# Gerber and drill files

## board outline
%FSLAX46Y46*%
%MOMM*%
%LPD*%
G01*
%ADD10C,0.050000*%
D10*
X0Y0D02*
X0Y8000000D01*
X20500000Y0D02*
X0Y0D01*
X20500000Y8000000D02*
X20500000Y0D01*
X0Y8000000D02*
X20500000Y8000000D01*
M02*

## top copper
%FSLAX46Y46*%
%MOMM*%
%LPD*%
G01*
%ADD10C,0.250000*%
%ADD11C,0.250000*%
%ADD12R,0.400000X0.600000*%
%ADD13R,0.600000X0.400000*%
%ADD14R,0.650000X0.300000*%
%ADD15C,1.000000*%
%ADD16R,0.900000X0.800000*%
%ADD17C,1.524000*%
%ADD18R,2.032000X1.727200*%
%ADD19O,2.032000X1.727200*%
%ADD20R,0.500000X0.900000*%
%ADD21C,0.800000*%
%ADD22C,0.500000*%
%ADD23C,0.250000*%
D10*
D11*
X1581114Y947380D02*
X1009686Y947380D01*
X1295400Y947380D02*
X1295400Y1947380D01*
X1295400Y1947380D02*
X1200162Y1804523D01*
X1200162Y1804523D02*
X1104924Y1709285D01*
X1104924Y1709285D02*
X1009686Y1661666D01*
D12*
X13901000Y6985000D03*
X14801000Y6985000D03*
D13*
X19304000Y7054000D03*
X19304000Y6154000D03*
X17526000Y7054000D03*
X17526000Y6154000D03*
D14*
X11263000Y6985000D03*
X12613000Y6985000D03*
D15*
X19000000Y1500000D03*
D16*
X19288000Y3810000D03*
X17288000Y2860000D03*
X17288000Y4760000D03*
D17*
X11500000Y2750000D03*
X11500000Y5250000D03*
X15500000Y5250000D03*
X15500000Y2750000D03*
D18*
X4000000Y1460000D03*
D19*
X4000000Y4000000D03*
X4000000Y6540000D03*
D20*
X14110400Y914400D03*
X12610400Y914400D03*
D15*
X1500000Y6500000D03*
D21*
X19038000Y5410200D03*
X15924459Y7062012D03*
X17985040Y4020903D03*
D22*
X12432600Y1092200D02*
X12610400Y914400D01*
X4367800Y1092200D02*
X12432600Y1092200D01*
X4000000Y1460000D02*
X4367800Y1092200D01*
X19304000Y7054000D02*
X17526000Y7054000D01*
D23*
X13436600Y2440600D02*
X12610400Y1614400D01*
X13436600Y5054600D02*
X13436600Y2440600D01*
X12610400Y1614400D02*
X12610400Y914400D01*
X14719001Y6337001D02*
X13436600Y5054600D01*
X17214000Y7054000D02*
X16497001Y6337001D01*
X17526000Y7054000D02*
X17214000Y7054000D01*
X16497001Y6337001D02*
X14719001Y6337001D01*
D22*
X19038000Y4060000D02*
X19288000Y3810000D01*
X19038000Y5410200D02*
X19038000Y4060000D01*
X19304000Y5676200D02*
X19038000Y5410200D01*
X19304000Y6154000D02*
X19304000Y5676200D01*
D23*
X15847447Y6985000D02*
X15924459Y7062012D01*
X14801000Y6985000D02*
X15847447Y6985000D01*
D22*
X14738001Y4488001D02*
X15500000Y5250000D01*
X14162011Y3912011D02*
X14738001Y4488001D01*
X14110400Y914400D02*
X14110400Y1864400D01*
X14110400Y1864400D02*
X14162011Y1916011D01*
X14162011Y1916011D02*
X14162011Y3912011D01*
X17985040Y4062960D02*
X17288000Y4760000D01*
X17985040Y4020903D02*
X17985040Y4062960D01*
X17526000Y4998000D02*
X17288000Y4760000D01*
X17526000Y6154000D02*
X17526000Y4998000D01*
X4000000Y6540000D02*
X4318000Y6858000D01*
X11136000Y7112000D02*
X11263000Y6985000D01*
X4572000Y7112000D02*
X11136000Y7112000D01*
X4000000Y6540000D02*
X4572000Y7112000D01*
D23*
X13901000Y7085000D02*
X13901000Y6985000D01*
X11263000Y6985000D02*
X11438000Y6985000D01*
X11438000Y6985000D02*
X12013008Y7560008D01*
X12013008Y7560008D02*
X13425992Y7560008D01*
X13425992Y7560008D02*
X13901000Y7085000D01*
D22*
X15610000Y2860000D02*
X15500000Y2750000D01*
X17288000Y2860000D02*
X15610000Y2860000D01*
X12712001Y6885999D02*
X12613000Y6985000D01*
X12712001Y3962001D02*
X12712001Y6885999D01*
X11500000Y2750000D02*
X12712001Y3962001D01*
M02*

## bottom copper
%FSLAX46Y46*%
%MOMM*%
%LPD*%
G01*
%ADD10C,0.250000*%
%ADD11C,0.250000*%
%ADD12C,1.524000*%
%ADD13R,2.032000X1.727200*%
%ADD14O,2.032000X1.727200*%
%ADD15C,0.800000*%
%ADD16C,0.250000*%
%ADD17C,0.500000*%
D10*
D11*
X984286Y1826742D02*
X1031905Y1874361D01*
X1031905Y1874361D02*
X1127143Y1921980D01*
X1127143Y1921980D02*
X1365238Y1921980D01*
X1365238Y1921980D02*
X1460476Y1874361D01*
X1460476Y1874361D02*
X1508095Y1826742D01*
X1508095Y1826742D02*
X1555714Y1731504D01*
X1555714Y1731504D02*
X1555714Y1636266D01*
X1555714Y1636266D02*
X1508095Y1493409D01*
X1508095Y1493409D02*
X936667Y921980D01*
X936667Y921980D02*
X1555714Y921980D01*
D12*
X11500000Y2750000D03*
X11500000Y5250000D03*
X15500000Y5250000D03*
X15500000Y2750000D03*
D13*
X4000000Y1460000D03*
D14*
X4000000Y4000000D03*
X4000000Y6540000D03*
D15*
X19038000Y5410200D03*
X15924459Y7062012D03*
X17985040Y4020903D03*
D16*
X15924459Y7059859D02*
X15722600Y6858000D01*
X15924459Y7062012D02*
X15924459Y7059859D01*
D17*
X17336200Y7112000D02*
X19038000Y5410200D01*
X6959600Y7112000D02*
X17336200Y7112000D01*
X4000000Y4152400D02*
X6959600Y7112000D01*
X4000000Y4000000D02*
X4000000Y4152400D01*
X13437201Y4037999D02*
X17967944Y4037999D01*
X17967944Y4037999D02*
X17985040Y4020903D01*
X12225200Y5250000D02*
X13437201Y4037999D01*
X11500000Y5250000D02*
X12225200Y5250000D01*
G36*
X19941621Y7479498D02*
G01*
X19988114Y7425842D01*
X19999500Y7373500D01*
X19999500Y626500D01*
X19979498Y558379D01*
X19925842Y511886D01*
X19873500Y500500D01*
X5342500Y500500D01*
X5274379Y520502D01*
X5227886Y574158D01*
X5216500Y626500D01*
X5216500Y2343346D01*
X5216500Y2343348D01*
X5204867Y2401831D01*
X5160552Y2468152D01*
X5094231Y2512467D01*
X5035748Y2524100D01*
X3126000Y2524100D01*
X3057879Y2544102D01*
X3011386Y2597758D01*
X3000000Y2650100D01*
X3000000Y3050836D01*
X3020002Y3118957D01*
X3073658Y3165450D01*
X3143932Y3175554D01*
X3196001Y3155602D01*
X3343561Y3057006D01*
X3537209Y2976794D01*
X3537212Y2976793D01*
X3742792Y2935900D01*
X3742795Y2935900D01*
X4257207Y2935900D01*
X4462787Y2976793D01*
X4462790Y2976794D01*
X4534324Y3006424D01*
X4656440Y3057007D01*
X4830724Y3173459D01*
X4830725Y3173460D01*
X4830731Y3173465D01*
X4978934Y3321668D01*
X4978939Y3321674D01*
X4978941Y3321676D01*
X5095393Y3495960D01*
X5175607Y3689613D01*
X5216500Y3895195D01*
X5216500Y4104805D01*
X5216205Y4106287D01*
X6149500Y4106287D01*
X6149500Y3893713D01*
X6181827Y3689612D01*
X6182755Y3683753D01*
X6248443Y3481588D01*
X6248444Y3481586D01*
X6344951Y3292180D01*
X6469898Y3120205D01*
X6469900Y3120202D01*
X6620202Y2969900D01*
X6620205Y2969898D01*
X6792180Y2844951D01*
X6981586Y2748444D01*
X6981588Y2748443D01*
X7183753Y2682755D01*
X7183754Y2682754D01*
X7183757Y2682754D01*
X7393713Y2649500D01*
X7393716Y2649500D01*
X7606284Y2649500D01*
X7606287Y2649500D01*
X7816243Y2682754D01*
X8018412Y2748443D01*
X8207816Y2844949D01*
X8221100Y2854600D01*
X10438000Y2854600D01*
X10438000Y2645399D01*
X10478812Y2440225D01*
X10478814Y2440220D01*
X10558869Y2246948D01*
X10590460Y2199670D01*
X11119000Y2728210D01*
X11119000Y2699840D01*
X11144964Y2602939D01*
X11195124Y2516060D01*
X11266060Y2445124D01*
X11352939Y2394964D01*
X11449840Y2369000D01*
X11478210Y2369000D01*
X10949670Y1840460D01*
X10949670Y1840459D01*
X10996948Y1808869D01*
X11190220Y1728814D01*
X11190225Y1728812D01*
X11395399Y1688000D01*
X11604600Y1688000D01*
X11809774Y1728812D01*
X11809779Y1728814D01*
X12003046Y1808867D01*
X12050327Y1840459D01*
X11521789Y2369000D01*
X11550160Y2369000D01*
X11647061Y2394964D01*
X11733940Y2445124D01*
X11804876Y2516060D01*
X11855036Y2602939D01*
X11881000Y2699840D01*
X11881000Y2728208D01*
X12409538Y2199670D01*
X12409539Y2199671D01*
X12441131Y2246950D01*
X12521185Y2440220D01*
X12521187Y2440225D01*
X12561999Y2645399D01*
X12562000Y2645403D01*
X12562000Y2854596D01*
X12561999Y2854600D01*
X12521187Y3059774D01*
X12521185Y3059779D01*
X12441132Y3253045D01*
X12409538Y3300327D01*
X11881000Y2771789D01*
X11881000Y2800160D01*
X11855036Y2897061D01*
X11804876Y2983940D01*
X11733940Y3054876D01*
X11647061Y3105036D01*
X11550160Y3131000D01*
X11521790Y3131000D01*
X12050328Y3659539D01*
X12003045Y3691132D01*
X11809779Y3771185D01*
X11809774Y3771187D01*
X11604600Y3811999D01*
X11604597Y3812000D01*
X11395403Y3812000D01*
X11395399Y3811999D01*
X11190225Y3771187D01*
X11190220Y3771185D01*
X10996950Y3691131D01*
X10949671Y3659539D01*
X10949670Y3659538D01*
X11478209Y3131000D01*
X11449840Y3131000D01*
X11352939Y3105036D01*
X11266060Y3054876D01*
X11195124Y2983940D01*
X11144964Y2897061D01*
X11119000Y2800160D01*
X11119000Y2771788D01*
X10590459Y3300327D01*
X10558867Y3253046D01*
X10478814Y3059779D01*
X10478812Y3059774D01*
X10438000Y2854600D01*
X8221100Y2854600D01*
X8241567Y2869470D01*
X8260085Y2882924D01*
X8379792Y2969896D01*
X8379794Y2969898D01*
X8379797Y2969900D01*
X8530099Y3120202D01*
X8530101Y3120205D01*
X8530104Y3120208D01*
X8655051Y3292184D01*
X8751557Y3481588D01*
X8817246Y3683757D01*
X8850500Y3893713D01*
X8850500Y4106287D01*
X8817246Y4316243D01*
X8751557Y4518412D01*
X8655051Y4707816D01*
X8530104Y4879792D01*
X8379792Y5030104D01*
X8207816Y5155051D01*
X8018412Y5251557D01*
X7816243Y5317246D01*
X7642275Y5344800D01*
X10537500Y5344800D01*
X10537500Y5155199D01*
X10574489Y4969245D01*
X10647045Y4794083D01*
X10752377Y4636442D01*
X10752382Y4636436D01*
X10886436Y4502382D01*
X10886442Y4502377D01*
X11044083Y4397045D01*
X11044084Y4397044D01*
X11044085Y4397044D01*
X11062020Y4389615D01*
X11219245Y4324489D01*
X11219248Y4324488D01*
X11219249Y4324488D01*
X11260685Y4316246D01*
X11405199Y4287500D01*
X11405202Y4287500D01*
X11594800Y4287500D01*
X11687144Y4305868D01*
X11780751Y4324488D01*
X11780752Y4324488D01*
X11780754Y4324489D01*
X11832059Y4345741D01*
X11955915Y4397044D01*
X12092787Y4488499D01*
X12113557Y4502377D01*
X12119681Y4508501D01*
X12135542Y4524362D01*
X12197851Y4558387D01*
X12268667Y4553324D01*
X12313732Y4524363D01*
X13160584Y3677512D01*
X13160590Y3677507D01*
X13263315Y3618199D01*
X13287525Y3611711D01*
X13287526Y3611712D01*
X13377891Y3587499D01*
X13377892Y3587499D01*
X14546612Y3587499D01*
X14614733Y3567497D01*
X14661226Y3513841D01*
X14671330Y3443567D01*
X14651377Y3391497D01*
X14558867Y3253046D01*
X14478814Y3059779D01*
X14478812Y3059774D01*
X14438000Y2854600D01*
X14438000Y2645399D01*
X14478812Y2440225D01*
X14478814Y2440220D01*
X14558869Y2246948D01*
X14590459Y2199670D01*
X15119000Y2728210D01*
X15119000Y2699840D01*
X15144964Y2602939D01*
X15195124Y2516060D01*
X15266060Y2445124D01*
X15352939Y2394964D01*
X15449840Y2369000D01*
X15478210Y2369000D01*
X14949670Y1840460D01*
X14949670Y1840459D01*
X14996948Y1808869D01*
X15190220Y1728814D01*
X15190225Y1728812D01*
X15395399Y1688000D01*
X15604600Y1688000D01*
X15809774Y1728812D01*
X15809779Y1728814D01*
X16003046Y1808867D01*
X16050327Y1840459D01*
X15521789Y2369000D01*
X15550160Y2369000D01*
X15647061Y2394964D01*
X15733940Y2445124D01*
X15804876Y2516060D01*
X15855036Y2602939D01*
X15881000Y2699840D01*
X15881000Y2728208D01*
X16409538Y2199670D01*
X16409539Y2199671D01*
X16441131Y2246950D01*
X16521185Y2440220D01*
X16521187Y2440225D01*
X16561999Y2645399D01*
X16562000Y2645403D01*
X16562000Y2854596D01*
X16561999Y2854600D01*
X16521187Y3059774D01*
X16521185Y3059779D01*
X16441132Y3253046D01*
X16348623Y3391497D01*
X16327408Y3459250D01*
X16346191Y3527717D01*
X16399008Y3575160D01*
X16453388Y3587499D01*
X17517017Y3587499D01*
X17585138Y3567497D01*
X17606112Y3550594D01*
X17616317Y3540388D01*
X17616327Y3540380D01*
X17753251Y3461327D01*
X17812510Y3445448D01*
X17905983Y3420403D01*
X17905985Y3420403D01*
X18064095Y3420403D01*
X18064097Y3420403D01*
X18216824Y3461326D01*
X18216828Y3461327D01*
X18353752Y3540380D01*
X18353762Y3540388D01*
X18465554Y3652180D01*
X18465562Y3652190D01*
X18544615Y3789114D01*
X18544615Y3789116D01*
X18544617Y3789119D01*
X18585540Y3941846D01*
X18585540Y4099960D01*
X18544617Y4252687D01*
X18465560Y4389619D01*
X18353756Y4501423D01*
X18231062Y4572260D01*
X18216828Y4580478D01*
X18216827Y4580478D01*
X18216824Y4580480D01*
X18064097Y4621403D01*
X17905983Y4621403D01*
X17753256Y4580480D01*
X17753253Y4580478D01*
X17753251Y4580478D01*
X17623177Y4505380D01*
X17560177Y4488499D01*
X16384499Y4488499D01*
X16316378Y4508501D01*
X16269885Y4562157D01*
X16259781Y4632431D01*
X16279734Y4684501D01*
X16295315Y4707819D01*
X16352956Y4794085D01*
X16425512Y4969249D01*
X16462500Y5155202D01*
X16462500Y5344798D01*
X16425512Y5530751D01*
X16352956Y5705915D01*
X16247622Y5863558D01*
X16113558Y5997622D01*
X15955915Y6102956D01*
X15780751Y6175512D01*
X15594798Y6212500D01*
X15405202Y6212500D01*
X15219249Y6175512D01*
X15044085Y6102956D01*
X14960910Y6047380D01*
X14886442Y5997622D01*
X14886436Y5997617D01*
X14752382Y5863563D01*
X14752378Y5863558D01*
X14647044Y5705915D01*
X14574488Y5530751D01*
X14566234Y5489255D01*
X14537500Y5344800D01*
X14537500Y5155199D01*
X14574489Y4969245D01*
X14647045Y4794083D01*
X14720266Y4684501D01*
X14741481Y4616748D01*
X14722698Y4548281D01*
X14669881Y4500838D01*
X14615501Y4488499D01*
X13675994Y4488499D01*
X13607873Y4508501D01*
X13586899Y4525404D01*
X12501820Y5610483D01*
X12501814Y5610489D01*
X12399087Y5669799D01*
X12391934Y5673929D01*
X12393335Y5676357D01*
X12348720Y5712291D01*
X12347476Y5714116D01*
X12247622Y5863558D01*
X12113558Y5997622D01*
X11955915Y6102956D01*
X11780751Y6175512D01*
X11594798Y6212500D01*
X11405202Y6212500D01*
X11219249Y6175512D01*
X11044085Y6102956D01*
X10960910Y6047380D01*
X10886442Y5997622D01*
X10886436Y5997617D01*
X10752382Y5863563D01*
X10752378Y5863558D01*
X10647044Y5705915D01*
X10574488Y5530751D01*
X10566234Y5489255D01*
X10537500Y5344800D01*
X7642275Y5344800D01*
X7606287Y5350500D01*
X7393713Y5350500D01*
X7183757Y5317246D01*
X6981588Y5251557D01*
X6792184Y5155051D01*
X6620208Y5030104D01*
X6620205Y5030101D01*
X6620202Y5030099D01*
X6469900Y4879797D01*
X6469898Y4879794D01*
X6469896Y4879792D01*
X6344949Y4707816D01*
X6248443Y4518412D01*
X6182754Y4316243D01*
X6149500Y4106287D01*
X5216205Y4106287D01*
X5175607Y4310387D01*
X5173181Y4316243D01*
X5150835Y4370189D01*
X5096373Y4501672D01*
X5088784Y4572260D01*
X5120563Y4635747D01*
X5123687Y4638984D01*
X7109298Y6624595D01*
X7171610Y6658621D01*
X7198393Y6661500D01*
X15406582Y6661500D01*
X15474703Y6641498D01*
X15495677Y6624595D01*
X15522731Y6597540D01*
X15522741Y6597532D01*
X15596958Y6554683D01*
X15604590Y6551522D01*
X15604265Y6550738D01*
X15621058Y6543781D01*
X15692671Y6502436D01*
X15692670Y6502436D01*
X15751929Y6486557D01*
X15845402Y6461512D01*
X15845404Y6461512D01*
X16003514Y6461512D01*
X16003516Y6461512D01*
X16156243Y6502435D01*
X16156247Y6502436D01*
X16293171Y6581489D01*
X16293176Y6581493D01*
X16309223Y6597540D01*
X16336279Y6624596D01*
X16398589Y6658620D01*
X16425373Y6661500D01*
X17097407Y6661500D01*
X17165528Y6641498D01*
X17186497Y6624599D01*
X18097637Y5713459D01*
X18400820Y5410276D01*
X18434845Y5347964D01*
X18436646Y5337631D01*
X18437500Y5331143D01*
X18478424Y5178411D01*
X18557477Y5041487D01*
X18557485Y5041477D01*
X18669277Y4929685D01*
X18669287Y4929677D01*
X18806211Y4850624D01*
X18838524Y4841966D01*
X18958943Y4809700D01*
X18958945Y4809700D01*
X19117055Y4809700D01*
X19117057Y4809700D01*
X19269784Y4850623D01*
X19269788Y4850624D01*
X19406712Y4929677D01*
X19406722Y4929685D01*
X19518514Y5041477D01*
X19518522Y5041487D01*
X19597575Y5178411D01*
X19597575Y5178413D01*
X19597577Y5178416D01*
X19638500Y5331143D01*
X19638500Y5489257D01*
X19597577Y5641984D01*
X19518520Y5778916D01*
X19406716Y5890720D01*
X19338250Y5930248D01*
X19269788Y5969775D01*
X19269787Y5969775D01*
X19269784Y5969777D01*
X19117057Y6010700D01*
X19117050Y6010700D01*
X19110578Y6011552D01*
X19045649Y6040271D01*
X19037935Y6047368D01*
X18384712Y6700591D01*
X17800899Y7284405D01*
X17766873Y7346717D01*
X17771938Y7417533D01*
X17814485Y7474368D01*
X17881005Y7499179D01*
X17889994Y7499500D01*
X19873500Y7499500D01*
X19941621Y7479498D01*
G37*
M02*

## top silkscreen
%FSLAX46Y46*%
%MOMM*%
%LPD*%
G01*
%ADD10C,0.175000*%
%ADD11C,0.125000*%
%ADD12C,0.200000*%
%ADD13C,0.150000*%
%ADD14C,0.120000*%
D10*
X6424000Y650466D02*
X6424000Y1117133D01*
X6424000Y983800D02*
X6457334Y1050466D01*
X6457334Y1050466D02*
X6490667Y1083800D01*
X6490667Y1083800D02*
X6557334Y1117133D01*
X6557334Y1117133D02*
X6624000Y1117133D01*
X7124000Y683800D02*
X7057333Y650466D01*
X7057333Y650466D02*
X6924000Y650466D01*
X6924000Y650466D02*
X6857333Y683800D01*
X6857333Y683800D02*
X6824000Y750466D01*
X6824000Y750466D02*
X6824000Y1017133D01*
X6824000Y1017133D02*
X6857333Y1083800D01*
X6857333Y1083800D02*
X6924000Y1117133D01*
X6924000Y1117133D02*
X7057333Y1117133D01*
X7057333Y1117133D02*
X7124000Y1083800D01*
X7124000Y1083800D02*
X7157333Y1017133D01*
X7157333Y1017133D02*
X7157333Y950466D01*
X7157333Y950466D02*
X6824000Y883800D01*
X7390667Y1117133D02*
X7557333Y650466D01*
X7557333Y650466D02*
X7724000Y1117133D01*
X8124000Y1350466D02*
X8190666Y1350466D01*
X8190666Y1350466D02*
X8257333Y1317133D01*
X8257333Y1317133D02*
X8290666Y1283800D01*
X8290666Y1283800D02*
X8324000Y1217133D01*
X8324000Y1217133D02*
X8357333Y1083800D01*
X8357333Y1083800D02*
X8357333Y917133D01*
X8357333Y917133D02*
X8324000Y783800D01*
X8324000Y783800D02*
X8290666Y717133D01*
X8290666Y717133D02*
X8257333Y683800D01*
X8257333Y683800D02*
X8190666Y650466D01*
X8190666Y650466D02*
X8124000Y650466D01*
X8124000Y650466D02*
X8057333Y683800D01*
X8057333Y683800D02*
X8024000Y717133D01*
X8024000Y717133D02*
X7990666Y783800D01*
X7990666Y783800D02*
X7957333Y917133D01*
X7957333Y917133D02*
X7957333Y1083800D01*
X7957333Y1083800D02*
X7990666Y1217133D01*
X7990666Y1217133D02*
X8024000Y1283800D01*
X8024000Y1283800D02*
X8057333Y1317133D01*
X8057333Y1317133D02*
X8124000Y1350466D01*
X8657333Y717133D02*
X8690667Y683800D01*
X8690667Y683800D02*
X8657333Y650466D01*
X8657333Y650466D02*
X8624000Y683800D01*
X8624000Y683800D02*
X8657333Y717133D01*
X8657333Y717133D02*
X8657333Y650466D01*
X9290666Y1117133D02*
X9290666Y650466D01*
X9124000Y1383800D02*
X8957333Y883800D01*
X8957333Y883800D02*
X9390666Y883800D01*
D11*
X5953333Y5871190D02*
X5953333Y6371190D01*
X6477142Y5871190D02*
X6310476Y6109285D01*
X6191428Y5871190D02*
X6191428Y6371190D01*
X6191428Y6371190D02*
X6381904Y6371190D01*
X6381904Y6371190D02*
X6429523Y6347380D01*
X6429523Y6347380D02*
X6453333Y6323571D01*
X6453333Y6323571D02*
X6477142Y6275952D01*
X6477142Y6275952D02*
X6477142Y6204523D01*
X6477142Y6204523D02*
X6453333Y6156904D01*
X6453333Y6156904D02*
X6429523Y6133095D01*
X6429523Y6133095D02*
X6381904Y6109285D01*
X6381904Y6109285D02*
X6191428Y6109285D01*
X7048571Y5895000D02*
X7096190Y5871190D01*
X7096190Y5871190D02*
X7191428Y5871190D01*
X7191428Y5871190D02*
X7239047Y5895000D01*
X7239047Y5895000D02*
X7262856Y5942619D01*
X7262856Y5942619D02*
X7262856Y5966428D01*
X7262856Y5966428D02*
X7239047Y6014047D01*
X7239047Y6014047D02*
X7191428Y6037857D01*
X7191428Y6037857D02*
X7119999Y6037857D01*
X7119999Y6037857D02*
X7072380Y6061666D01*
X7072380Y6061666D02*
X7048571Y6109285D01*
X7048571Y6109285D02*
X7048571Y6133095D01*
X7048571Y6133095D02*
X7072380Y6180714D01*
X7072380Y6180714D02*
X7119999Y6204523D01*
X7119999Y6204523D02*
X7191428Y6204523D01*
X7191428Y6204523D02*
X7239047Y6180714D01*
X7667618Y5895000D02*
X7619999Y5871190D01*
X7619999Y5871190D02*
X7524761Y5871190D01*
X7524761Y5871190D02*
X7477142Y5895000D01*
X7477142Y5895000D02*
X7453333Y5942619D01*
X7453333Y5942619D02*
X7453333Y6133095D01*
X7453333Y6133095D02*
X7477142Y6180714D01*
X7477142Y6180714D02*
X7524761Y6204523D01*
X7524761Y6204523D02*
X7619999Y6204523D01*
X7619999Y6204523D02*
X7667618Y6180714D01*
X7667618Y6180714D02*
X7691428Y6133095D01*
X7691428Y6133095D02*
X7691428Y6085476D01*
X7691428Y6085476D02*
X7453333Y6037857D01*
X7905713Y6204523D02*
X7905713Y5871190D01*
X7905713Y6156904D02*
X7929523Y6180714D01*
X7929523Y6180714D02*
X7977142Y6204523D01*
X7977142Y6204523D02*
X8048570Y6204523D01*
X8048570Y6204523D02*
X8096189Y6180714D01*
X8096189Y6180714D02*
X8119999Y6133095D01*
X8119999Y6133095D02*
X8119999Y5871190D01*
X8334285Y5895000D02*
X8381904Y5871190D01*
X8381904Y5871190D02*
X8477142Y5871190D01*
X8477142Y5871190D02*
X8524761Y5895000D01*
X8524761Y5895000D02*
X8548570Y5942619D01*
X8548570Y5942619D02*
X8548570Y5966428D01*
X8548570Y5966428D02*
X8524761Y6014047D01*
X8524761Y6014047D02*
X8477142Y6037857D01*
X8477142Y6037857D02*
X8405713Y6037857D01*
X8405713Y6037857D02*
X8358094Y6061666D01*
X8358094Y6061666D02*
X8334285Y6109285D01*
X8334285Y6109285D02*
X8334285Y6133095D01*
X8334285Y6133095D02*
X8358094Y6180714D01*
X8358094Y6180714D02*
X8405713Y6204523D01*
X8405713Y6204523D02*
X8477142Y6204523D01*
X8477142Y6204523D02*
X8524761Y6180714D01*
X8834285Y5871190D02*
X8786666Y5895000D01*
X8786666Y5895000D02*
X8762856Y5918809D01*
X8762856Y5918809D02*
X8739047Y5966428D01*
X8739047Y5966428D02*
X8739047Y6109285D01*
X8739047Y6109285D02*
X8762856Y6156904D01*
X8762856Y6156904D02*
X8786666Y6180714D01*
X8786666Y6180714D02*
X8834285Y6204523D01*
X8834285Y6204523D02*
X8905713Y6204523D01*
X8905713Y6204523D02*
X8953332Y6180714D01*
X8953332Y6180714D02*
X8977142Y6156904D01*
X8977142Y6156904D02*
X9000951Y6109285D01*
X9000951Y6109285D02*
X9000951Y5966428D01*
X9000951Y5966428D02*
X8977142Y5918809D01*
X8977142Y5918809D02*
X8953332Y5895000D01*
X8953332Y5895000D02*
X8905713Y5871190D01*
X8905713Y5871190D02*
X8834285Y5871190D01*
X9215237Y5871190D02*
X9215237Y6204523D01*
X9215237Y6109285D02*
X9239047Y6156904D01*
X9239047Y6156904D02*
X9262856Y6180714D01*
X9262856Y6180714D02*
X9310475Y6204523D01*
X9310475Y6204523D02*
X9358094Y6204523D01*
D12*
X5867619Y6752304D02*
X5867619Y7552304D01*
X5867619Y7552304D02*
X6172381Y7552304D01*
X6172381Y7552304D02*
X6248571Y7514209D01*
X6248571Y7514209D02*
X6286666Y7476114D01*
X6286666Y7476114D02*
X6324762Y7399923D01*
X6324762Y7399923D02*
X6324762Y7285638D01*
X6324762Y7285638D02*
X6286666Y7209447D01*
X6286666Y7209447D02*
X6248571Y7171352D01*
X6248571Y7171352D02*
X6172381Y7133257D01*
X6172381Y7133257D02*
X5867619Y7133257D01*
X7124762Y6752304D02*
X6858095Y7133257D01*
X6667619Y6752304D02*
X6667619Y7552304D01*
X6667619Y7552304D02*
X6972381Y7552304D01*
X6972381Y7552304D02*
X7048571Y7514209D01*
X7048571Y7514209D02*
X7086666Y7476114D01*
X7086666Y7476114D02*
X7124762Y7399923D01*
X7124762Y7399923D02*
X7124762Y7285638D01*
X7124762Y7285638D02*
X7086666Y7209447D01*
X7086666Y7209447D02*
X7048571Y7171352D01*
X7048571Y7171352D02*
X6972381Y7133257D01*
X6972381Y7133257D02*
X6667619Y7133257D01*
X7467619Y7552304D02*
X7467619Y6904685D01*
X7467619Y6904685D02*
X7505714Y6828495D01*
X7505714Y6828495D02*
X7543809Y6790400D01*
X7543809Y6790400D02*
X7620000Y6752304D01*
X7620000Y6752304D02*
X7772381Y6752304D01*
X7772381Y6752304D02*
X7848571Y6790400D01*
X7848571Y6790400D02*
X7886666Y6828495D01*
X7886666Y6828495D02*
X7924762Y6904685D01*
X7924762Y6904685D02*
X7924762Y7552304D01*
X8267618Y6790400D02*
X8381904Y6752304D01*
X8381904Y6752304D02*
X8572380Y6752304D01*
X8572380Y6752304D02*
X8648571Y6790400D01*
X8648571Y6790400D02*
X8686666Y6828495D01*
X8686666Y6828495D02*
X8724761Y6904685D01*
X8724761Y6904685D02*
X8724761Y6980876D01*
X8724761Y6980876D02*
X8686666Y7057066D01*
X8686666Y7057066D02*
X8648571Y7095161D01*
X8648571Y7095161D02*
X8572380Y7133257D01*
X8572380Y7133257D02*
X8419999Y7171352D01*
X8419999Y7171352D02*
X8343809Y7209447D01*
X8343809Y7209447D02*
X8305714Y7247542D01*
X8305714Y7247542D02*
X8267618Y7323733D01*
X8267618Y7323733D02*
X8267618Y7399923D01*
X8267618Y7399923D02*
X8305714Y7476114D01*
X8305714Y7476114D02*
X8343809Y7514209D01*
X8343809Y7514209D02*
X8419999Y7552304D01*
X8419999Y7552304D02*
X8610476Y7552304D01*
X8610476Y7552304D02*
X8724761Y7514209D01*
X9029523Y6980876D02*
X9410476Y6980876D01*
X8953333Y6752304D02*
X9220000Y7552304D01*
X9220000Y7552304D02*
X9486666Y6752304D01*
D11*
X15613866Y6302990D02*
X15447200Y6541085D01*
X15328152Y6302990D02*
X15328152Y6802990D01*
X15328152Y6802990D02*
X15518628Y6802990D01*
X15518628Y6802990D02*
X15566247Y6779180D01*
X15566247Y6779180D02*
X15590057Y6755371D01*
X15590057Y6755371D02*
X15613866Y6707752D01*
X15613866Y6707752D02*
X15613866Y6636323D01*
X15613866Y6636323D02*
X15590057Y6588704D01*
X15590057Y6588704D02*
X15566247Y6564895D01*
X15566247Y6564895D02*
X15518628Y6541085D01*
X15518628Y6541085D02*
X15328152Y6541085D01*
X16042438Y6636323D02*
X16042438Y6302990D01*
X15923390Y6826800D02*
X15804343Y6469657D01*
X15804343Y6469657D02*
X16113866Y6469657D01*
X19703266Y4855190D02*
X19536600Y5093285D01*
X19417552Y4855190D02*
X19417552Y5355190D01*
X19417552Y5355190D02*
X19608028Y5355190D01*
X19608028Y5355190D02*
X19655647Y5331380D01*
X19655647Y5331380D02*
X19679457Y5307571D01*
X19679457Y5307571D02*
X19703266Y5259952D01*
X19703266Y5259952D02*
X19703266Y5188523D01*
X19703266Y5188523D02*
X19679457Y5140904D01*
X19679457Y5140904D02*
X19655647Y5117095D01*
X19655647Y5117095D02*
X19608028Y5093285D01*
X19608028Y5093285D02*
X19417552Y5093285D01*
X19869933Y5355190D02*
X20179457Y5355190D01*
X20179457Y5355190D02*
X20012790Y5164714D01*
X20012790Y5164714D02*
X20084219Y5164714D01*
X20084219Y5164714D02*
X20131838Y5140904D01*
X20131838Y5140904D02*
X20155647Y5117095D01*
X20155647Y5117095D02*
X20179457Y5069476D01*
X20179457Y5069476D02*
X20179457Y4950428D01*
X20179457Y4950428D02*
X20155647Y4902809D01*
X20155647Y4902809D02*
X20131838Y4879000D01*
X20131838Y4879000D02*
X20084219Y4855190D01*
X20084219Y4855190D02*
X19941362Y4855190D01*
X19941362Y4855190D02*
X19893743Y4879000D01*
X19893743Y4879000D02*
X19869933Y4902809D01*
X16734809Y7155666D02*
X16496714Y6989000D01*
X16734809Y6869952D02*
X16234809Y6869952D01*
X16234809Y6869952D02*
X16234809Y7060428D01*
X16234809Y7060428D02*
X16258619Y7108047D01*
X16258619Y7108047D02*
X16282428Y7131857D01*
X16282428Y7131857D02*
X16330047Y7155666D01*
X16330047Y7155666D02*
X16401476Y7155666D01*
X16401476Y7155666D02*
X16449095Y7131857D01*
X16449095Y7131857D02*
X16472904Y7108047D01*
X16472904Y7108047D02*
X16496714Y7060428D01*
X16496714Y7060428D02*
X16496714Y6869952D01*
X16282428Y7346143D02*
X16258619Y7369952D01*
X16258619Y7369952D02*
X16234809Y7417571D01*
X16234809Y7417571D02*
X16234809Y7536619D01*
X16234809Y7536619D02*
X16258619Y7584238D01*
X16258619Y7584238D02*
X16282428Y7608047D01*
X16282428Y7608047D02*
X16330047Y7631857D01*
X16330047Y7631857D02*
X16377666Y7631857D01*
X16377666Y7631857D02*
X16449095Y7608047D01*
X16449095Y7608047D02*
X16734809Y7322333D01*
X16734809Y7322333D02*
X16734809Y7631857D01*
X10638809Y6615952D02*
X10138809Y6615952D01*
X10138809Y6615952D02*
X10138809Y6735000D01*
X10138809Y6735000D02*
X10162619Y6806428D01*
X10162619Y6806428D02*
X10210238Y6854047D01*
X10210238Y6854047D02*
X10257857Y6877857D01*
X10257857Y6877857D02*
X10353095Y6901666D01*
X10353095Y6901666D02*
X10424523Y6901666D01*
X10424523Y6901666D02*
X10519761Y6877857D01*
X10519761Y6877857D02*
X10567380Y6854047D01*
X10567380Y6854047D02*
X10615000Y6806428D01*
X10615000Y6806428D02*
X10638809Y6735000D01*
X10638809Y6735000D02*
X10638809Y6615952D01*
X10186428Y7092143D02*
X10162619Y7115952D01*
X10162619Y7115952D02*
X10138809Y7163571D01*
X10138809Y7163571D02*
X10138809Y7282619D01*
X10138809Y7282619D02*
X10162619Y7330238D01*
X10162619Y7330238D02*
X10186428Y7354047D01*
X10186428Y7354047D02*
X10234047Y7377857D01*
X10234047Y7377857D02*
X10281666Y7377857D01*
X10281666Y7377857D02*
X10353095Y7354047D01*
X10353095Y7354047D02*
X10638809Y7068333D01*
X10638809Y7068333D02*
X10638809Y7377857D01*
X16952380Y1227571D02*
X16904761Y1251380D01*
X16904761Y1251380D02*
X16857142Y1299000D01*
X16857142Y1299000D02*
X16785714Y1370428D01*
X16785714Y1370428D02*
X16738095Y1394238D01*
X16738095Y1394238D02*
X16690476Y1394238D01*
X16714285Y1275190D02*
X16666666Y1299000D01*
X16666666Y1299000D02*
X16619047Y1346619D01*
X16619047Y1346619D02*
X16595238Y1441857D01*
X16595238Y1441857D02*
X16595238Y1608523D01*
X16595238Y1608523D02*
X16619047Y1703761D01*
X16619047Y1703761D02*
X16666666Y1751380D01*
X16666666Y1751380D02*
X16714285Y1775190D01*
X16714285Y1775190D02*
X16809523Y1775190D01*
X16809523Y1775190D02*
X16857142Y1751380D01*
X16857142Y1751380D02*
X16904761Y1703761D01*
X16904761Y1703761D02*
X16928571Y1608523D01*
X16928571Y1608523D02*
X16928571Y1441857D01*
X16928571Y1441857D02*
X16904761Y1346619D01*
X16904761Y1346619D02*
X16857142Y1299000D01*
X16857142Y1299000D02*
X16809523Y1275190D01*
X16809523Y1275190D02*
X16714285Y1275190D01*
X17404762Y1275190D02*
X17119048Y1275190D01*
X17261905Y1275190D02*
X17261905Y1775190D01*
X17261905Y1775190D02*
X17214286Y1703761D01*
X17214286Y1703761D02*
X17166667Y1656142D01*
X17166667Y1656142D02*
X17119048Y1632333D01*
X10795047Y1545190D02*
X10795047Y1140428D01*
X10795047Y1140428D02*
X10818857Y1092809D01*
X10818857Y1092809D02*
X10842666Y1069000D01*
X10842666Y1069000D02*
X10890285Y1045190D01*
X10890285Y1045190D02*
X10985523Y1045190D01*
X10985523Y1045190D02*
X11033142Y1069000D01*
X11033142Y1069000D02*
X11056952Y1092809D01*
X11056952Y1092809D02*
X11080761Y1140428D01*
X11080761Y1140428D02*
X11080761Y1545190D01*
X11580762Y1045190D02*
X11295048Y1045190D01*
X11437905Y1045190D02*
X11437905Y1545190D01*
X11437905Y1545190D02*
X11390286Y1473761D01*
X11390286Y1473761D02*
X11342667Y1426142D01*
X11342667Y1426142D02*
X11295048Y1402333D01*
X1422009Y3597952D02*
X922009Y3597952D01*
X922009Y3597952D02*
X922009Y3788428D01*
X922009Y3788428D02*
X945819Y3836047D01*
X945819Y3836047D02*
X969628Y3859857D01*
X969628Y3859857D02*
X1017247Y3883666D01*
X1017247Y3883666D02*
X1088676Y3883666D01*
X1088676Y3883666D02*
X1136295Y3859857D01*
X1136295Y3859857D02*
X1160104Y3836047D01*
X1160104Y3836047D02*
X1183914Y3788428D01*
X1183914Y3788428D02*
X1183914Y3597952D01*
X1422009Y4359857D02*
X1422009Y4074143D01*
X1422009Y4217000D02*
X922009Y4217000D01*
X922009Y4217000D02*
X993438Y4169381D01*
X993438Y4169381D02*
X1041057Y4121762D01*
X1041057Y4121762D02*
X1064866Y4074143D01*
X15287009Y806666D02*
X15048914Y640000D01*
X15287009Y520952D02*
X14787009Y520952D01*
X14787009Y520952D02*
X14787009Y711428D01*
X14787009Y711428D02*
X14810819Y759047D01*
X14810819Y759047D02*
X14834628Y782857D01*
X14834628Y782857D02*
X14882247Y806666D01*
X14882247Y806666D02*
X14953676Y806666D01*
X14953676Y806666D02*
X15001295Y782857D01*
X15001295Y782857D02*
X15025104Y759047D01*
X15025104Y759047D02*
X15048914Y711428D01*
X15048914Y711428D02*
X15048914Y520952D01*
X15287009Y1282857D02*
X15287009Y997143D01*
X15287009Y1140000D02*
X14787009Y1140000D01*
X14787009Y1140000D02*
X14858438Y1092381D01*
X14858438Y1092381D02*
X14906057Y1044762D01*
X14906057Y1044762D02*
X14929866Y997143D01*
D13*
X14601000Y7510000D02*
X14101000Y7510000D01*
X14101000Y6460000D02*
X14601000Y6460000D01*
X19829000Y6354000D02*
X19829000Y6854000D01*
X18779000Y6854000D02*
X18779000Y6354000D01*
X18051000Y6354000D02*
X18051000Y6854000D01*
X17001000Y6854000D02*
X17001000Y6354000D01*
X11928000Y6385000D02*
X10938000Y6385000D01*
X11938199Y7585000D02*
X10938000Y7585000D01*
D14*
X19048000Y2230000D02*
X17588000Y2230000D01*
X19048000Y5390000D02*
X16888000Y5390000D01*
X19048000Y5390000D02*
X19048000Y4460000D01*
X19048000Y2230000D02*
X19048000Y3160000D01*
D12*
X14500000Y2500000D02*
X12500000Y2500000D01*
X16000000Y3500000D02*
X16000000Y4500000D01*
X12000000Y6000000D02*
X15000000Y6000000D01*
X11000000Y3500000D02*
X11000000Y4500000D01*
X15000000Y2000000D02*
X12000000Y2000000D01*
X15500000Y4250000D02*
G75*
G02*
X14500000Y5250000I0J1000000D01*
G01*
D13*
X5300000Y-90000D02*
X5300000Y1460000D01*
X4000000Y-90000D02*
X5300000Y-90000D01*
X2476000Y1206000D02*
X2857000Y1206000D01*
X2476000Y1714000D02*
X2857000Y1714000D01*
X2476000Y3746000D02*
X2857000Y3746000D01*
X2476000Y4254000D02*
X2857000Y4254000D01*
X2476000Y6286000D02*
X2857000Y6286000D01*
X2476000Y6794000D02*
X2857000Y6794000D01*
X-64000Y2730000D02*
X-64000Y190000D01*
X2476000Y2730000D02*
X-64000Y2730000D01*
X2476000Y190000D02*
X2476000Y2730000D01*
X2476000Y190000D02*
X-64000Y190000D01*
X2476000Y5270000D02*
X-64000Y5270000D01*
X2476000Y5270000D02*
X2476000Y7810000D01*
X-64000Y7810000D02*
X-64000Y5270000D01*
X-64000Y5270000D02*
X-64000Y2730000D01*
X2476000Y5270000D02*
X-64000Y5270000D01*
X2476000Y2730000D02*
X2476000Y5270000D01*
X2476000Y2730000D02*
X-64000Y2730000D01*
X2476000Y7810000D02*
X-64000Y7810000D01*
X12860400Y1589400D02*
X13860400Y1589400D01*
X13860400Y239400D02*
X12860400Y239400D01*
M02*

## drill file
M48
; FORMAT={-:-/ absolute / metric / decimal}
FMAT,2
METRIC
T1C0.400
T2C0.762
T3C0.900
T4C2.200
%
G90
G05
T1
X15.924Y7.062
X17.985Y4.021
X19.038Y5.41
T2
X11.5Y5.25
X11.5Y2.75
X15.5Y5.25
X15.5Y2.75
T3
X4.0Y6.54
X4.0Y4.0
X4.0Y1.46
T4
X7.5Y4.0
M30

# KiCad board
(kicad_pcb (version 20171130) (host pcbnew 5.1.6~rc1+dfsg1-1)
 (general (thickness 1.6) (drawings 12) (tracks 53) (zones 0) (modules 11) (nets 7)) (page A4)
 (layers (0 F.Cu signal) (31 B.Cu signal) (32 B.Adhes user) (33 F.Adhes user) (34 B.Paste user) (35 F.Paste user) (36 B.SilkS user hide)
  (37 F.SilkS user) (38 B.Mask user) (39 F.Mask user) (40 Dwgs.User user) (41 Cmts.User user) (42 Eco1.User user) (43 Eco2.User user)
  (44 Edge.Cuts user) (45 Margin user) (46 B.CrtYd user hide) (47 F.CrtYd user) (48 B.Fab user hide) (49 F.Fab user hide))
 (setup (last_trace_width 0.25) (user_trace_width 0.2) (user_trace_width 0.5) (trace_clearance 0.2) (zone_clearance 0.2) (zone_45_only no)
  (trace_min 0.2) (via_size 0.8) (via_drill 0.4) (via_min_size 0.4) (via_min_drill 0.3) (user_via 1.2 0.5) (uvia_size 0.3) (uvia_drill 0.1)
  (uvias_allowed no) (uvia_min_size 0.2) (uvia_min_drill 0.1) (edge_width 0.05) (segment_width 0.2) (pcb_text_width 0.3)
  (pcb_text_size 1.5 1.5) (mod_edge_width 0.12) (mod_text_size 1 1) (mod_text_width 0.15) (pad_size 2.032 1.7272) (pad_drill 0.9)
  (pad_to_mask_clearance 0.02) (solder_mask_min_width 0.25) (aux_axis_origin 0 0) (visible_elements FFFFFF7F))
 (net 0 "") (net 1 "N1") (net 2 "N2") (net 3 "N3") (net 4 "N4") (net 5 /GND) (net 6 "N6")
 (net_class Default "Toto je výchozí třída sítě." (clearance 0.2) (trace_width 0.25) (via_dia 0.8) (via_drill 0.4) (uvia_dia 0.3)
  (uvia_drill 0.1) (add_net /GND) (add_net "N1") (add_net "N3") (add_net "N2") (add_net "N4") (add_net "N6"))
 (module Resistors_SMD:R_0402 (layer F.Cu) (at 14.351 -6.985)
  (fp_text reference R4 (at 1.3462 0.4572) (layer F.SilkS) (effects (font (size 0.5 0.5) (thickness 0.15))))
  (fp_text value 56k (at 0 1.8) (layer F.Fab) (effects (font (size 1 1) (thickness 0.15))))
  (fp_line (start 0.25 -0.525) (end -0.25 -0.525) (layer F.SilkS) (width 0.15))
  (fp_line (start -0.25 0.525) (end 0.25 0.525) (layer F.SilkS) (width 0.15))
  (pad 1 smd rect (at -0.45 0) (size 0.4 0.6) (layers F.Cu F.Paste F.Mask) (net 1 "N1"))
  (pad 2 smd rect (at 0.45 0) (size 0.4 0.6) (layers F.Cu F.Paste F.Mask) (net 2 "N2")))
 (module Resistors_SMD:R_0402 (layer F.Cu) (at 19.304 -6.604 90)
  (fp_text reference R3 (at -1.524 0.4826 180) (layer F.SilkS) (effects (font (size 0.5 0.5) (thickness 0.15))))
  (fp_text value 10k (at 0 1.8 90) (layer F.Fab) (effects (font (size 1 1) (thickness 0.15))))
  (fp_line (start -0.25 0.525) (end 0.25 0.525) (layer F.SilkS) (width 0.15))
  (fp_line (start 0.25 -0.525) (end -0.25 -0.525) (layer F.SilkS) (width 0.15))
  (pad 2 smd rect (at 0.45 0 90) (size 0.4 0.6) (layers F.Cu F.Paste F.Mask) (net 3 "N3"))
  (pad 1 smd rect (at -0.45 0 90) (size 0.4 0.6) (layers F.Cu F.Paste F.Mask) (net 2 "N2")))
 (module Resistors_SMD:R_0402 (layer F.Cu) (at 17.526 -6.604 270)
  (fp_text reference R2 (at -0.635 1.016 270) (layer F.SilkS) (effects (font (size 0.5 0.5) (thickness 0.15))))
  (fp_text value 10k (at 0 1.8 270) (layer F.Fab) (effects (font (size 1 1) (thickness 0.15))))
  (fp_line (start 0.25 -0.525) (end -0.25 -0.525) (layer F.SilkS) (width 0.15))
  (fp_line (start -0.25 0.525) (end 0.25 0.525) (layer F.SilkS) (width 0.15))
  (pad 1 smd rect (at -0.45 0 270) (size 0.4 0.6) (layers F.Cu F.Paste F.Mask) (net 3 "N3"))
  (pad 2 smd rect (at 0.45 0 270) (size 0.4 0.6) (layers F.Cu F.Paste F.Mask) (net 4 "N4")))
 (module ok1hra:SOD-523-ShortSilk (layer F.Cu) (at 11.938 -6.985)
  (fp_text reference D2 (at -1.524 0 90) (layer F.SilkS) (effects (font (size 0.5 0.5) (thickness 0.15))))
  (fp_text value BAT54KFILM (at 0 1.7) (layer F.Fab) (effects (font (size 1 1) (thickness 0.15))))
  (fp_line (start -0.01 0.6) (end -1 0.6) (layer F.SilkS) (width 0.15))
  (fp_line (start 0.000199 -0.6) (end -1 -0.6) (layer F.SilkS) (width 0.15))
  (pad 1 smd rect (at -0.675 0 180) (size 0.65 0.3) (layers F.Cu F.Paste F.Mask) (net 1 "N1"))
  (pad 2 smd rect (at 0.675 0 180) (size 0.65 0.3) (layers F.Cu F.Paste F.Mask) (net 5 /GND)))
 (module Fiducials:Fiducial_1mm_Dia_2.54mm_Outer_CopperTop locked (layer F.Cu) (at 19 -1.5)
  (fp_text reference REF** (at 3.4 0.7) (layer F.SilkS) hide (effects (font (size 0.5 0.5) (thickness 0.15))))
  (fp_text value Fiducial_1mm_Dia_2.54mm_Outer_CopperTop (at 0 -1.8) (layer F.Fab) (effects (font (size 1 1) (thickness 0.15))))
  (pad ~ smd circle (at 0 0) (size 1 1) (layers F.Cu F.Mask) (solder_mask_margin 0.77) (clearance 0.77)))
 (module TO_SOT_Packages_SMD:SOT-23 (layer F.Cu) (at 18.288 -3.81)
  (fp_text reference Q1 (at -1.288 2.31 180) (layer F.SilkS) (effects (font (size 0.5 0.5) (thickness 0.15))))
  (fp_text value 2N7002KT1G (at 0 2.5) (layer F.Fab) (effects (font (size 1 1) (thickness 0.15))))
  (fp_line (start 0.76 1.58) (end -0.7 1.58) (layer F.SilkS) (width 0.12))
  (fp_line (start 0.76 -1.58) (end -1.4 -1.58) (layer F.SilkS) (width 0.12))
  (fp_line (start 0.76 -1.58) (end 0.76 -0.65) (layer F.SilkS) (width 0.12))
  (fp_line (start 0.76 1.58) (end 0.76 0.65) (layer F.SilkS) (width 0.12))
  (pad 3 smd rect (at 1 0) (size 0.9 0.8) (layers F.Cu F.Paste F.Mask) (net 2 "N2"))
  (pad 2 smd rect (at -1 0.95) (size 0.9 0.8) (layers F.Cu F.Paste F.Mask) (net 5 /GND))
  (pad 1 smd rect (at -1 -0.95) (size 0.9 0.8) (layers F.Cu F.Paste F.Mask) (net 4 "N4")))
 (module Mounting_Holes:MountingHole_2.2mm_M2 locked (layer F.Cu) (at 7.5 -4)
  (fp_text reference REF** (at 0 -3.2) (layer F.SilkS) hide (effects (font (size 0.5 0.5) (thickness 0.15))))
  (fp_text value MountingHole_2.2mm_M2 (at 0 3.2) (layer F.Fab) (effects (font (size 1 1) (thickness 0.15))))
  (pad 1 np_thru_hole circle (at 0 0) (size 2.2 2.2) (drill 2.2) (layers *.Cu *.Mask)))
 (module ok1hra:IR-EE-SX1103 (layer F.Cu) (at 13.5 -4 180)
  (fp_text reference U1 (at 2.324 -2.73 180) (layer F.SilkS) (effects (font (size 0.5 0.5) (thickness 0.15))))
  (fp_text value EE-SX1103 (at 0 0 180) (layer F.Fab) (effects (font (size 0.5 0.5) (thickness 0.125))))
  (fp_line (start -1 -1.5) (end 1 -1.5) (layer F.SilkS) (width 0.2))
  (fp_line (start -2.5 -0.5) (end -2.5 0.5) (layer F.SilkS) (width 0.2))
  (fp_line (start 1.5 2) (end -1.5 2) (layer F.SilkS) (width 0.2))
  (fp_line (start 2.5 -0.5) (end 2.5 0.5) (layer F.SilkS) (width 0.2))
  (fp_line (start -1.5 -2) (end 1.5 -2) (layer F.SilkS) (width 0.2))
  (fp_arc (start -2 1.25) (end -1 1.25) (angle -90) (layer F.SilkS) (width 0.2))
  (pad 3 thru_hole circle (at 2 -1.25 180) (size 1.524 1.524) (drill 0.762) (layers *.Cu *.Mask) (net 5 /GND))
  (pad 4 thru_hole circle (at 2 1.25 180) (size 1.524 1.524) (drill 0.762) (layers *.Cu *.Mask) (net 4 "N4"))
  (pad 1 thru_hole circle (at -2 1.25 180) (size 1.524 1.524) (drill 0.762) (layers *.Cu *.Mask) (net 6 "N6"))
  (pad 2 thru_hole circle (at -2 -1.25 180) (size 1.524 1.524) (drill 0.762) (layers *.Cu *.Mask) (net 5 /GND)))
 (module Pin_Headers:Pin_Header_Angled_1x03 (layer F.Cu) (at 4 -1.46 180)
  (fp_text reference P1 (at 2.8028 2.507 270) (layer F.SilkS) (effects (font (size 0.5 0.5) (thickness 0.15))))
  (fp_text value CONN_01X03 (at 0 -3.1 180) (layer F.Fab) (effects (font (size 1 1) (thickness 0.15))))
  (fp_line (start -1.3 -1.55) (end -1.3 0) (layer F.SilkS) (width 0.15))
  (fp_line (start 0 -1.55) (end -1.3 -1.55) (layer F.SilkS) (width 0.15))
  (fp_line (start 1.524 -0.254) (end 1.143 -0.254) (layer F.SilkS) (width 0.15))
  (fp_line (start 1.524 0.254) (end 1.143 0.254) (layer F.SilkS) (width 0.15))
  (fp_line (start 1.524 2.286) (end 1.143 2.286) (layer F.SilkS) (width 0.15))
  (fp_line (start 1.524 2.794) (end 1.143 2.794) (layer F.SilkS) (width 0.15))
  (fp_line (start 1.524 4.826) (end 1.143 4.826) (layer F.SilkS) (width 0.15))
  (fp_line (start 1.524 5.334) (end 1.143 5.334) (layer F.SilkS) (width 0.15))
  (fp_line (start 4.064 1.27) (end 4.064 -1.27) (layer F.SilkS) (width 0.15))
  (fp_line (start 1.524 1.27) (end 4.064 1.27) (layer F.SilkS) (width 0.15))
  (fp_line (start 1.524 -1.27) (end 1.524 1.27) (layer F.SilkS) (width 0.15))
  (fp_line (start 1.524 -1.27) (end 4.064 -1.27) (layer F.SilkS) (width 0.15))
  (fp_line (start 1.524 3.81) (end 4.064 3.81) (layer F.SilkS) (width 0.15))
  (fp_line (start 1.524 3.81) (end 1.524 6.35) (layer F.SilkS) (width 0.15))
  (fp_line (start 4.064 6.35) (end 4.064 3.81) (layer F.SilkS) (width 0.15))
  (fp_line (start 4.064 3.81) (end 4.064 1.27) (layer F.SilkS) (width 0.15))
  (fp_line (start 1.524 3.81) (end 4.064 3.81) (layer F.SilkS) (width 0.15))
  (fp_line (start 1.524 1.27) (end 1.524 3.81) (layer F.SilkS) (width 0.15))
  (fp_line (start 1.524 1.27) (end 4.064 1.27) (layer F.SilkS) (width 0.15))
  (fp_line (start 1.524 6.35) (end 4.064 6.35) (layer F.SilkS) (width 0.15))
  (pad 1 thru_hole rect (at 0 0 180) (size 2.032 1.7272) (drill 0.9) (layers *.Cu *.Mask) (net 3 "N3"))
  (pad 2 thru_hole oval (at 0 2.54 180) (size 2.032 1.7272) (drill 0.9) (layers *.Cu *.Mask) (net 2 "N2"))
  (pad 3 thru_hole oval (at 0 5.08 180) (size 2.032 1.7272) (drill 0.9) (layers *.Cu *.Mask) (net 1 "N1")))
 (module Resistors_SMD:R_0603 (layer F.Cu) (at 13.3604 -0.9144 180)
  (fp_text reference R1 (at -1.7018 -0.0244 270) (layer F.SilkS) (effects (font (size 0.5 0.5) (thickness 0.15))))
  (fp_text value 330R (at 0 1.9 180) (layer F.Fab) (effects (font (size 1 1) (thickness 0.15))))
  (fp_line (start 0.5 0.675) (end -0.5 0.675) (layer F.SilkS) (width 0.15))
  (fp_line (start -0.5 -0.675) (end 0.5 -0.675) (layer F.SilkS) (width 0.15))
  (pad 1 smd rect (at -0.75 0 180) (size 0.5 0.9) (layers F.Cu F.Paste F.Mask) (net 6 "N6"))
  (pad 2 smd rect (at 0.75 0 180) (size 0.5 0.9) (layers F.Cu F.Paste F.Mask) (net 3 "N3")))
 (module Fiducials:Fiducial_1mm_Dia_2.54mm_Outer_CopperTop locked (layer F.Cu) (at 1.5 -6.5)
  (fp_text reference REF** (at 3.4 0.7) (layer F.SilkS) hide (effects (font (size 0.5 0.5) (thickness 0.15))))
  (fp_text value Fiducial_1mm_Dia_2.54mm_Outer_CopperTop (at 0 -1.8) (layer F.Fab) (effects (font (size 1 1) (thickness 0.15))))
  (pad ~ smd circle (at 0 0) (size 1 1) (layers F.Cu F.Mask) (solder_mask_margin 0.77) (clearance 0.77)))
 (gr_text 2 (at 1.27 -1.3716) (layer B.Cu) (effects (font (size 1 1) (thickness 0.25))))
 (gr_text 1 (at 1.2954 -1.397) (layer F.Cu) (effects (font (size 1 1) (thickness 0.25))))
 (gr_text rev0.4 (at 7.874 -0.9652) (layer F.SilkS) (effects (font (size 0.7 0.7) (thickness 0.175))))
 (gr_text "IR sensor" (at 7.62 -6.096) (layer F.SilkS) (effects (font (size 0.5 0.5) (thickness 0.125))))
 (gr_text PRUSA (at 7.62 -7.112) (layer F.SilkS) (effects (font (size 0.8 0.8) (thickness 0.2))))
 (gr_line (start 0 0) (end 0 -8) (layer Edge.Cuts) (width 0.05))
 (gr_line (start 20.5 0) (end 0 0) (layer Edge.Cuts) (width 0.05))
 (gr_line (start 20.5 -8) (end 20.5 0) (layer Edge.Cuts) (width 0.05))
 (gr_line (start 0 -8) (end 20.5 -8) (layer Edge.Cuts) (width 0.05))
 (segment (start 12.4326 -1.0922) (end 12.6104 -0.9144) (width 0.5) (layer F.Cu) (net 3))
 (segment (start 4.3678 -1.0922) (end 12.4326 -1.0922) (width 0.5) (layer F.Cu) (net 3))
 (segment (start 4 -1.46) (end 4.3678 -1.0922) (width 0.5) (layer F.Cu) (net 3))
 (segment (start 19.304 -7.054) (end 17.526 -7.054) (width 0.5) (layer F.Cu) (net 3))
 (segment (start 13.4366 -2.4406) (end 12.6104 -1.6144) (width 0.25) (layer F.Cu) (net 3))
 (segment (start 13.4366 -5.0546) (end 13.4366 -2.4406) (width 0.25) (layer F.Cu) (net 3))
 (segment (start 12.6104 -1.6144) (end 12.6104 -0.9144) (width 0.25) (layer F.Cu) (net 3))
 (segment (start 14.719001 -6.337001) (end 13.4366 -5.0546) (width 0.25) (layer F.Cu) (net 3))
 (segment (start 17.214 -7.054) (end 16.497001 -6.337001) (width 0.25) (layer F.Cu) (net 3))
 (segment (start 17.526 -7.054) (end 17.214 -7.054) (width 0.25) (layer F.Cu) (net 3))
 (segment (start 16.497001 -6.337001) (end 14.719001 -6.337001) (width 0.25) (layer F.Cu) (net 3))
 (segment (start 19.038 -4.06) (end 19.288 -3.81) (width 0.5) (layer F.Cu) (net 2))
 (segment (start 19.038 -5.4102) (end 19.038 -4.06) (width 0.5) (layer F.Cu) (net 2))
 (via (at 19.038 -5.4102) (size 0.8) (drill 0.4) (layers F.Cu B.Cu) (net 2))
 (segment (start 19.304 -5.6762) (end 19.038 -5.4102) (width 0.5) (layer F.Cu) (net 2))
 (segment (start 19.304 -6.154) (end 19.304 -5.6762) (width 0.5) (layer F.Cu) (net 2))
 (via (at 15.924459 -7.062012) (size 0.8) (drill 0.4) (layers F.Cu B.Cu) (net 2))
 (segment (start 15.847447 -6.985) (end 15.924459 -7.062012) (width 0.25) (layer F.Cu) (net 2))
 (segment (start 14.801 -6.985) (end 15.847447 -6.985) (width 0.25) (layer F.Cu) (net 2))
 (segment (start 15.924459 -7.059859) (end 15.7226 -6.858) (width 0.25) (layer B.Cu) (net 2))
 (segment (start 15.924459 -7.062012) (end 15.924459 -7.059859) (width 0.25) (layer B.Cu) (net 2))
 (segment (start 17.3362 -7.112) (end 19.038 -5.4102) (width 0.5) (layer B.Cu) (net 2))
 (segment (start 6.9596 -7.112) (end 17.3362 -7.112) (width 0.5) (layer B.Cu) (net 2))
 (segment (start 4 -4.1524) (end 6.9596 -7.112) (width 0.5) (layer B.Cu) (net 2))
 (segment (start 4 -4) (end 4 -4.1524) (width 0.5) (layer B.Cu) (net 2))
 (segment (start 14.738001 -4.488001) (end 15.5 -5.25) (width 0.5) (layer F.Cu) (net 6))
 (segment (start 14.162011 -3.912011) (end 14.738001 -4.488001) (width 0.5) (layer F.Cu) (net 6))
 (segment (start 14.1104 -0.9144) (end 14.1104 -1.8644) (width 0.5) (layer F.Cu) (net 6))
 (segment (start 14.1104 -1.8644) (end 14.162011 -1.916011) (width 0.5) (layer F.Cu) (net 6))
 (segment (start 14.162011 -1.916011) (end 14.162011 -3.912011) (width 0.5) (layer F.Cu) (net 6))
 (via (at 17.98504 -4.020903) (size 0.8) (drill 0.4) (layers F.Cu B.Cu) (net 4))
 (segment (start 17.98504 -4.06296) (end 17.288 -4.76) (width 0.5) (layer F.Cu) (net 4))
 (segment (start 17.98504 -4.020903) (end 17.98504 -4.06296) (width 0.5) (layer F.Cu) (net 4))
 (segment (start 17.526 -4.998) (end 17.288 -4.76) (width 0.5) (layer F.Cu) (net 4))
 (segment (start 17.526 -6.154) (end 17.526 -4.998) (width 0.5) (layer F.Cu) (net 4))
 (segment (start 13.437201 -4.037999) (end 17.967944 -4.037999) (width 0.5) (layer B.Cu) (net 4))
 (segment (start 17.967944 -4.037999) (end 17.98504 -4.020903) (width 0.5) (layer B.Cu) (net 4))
 (segment (start 12.2252 -5.25) (end 13.437201 -4.037999) (width 0.5) (layer B.Cu) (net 4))
 (segment (start 11.5 -5.25) (end 12.2252 -5.25) (width 0.5) (layer B.Cu) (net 4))
 (segment (start 4 -6.54) (end 4.318 -6.858) (width 0.5) (layer F.Cu) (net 1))
 (segment (start 11.136 -7.112) (end 11.263 -6.985) (width 0.5) (layer F.Cu) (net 1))
 (segment (start 4.572 -7.112) (end 11.136 -7.112) (width 0.5) (layer F.Cu) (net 1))
 (segment (start 4 -6.54) (end 4.572 -7.112) (width 0.5) (layer F.Cu) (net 1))
 (segment (start 13.901 -7.085) (end 13.901 -6.985) (width 0.25) (layer F.Cu) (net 1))
 (segment (start 11.263 -6.985) (end 11.438 -6.985) (width 0.25) (layer F.Cu) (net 1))
 (segment (start 11.438 -6.985) (end 12.013008 -7.560008) (width 0.25) (layer F.Cu) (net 1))
 (segment (start 12.013008 -7.560008) (end 13.425992 -7.560008) (width 0.25) (layer F.Cu) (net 1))
 (segment (start 13.425992 -7.560008) (end 13.901 -7.085) (width 0.25) (layer F.Cu) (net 1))
 (segment (start 15.61 -2.86) (end 15.5 -2.75) (width 0.5) (layer F.Cu) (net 5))
 (segment (start 17.288 -2.86) (end 15.61 -2.86) (width 0.5) (layer F.Cu) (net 5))
 (segment (start 12.712001 -6.885999) (end 12.613 -6.985) (width 0.5) (layer F.Cu) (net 5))
 (segment (start 12.712001 -3.962001) (end 12.712001 -6.885999) (width 0.5) (layer F.Cu) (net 5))
 (segment (start 11.5 -2.75) (end 12.712001 -3.962001) (width 0.5) (layer F.Cu) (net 5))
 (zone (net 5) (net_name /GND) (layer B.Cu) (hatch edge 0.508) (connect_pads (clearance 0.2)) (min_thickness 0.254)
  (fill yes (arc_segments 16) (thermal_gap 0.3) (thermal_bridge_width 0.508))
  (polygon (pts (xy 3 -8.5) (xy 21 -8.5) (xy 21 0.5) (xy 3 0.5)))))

